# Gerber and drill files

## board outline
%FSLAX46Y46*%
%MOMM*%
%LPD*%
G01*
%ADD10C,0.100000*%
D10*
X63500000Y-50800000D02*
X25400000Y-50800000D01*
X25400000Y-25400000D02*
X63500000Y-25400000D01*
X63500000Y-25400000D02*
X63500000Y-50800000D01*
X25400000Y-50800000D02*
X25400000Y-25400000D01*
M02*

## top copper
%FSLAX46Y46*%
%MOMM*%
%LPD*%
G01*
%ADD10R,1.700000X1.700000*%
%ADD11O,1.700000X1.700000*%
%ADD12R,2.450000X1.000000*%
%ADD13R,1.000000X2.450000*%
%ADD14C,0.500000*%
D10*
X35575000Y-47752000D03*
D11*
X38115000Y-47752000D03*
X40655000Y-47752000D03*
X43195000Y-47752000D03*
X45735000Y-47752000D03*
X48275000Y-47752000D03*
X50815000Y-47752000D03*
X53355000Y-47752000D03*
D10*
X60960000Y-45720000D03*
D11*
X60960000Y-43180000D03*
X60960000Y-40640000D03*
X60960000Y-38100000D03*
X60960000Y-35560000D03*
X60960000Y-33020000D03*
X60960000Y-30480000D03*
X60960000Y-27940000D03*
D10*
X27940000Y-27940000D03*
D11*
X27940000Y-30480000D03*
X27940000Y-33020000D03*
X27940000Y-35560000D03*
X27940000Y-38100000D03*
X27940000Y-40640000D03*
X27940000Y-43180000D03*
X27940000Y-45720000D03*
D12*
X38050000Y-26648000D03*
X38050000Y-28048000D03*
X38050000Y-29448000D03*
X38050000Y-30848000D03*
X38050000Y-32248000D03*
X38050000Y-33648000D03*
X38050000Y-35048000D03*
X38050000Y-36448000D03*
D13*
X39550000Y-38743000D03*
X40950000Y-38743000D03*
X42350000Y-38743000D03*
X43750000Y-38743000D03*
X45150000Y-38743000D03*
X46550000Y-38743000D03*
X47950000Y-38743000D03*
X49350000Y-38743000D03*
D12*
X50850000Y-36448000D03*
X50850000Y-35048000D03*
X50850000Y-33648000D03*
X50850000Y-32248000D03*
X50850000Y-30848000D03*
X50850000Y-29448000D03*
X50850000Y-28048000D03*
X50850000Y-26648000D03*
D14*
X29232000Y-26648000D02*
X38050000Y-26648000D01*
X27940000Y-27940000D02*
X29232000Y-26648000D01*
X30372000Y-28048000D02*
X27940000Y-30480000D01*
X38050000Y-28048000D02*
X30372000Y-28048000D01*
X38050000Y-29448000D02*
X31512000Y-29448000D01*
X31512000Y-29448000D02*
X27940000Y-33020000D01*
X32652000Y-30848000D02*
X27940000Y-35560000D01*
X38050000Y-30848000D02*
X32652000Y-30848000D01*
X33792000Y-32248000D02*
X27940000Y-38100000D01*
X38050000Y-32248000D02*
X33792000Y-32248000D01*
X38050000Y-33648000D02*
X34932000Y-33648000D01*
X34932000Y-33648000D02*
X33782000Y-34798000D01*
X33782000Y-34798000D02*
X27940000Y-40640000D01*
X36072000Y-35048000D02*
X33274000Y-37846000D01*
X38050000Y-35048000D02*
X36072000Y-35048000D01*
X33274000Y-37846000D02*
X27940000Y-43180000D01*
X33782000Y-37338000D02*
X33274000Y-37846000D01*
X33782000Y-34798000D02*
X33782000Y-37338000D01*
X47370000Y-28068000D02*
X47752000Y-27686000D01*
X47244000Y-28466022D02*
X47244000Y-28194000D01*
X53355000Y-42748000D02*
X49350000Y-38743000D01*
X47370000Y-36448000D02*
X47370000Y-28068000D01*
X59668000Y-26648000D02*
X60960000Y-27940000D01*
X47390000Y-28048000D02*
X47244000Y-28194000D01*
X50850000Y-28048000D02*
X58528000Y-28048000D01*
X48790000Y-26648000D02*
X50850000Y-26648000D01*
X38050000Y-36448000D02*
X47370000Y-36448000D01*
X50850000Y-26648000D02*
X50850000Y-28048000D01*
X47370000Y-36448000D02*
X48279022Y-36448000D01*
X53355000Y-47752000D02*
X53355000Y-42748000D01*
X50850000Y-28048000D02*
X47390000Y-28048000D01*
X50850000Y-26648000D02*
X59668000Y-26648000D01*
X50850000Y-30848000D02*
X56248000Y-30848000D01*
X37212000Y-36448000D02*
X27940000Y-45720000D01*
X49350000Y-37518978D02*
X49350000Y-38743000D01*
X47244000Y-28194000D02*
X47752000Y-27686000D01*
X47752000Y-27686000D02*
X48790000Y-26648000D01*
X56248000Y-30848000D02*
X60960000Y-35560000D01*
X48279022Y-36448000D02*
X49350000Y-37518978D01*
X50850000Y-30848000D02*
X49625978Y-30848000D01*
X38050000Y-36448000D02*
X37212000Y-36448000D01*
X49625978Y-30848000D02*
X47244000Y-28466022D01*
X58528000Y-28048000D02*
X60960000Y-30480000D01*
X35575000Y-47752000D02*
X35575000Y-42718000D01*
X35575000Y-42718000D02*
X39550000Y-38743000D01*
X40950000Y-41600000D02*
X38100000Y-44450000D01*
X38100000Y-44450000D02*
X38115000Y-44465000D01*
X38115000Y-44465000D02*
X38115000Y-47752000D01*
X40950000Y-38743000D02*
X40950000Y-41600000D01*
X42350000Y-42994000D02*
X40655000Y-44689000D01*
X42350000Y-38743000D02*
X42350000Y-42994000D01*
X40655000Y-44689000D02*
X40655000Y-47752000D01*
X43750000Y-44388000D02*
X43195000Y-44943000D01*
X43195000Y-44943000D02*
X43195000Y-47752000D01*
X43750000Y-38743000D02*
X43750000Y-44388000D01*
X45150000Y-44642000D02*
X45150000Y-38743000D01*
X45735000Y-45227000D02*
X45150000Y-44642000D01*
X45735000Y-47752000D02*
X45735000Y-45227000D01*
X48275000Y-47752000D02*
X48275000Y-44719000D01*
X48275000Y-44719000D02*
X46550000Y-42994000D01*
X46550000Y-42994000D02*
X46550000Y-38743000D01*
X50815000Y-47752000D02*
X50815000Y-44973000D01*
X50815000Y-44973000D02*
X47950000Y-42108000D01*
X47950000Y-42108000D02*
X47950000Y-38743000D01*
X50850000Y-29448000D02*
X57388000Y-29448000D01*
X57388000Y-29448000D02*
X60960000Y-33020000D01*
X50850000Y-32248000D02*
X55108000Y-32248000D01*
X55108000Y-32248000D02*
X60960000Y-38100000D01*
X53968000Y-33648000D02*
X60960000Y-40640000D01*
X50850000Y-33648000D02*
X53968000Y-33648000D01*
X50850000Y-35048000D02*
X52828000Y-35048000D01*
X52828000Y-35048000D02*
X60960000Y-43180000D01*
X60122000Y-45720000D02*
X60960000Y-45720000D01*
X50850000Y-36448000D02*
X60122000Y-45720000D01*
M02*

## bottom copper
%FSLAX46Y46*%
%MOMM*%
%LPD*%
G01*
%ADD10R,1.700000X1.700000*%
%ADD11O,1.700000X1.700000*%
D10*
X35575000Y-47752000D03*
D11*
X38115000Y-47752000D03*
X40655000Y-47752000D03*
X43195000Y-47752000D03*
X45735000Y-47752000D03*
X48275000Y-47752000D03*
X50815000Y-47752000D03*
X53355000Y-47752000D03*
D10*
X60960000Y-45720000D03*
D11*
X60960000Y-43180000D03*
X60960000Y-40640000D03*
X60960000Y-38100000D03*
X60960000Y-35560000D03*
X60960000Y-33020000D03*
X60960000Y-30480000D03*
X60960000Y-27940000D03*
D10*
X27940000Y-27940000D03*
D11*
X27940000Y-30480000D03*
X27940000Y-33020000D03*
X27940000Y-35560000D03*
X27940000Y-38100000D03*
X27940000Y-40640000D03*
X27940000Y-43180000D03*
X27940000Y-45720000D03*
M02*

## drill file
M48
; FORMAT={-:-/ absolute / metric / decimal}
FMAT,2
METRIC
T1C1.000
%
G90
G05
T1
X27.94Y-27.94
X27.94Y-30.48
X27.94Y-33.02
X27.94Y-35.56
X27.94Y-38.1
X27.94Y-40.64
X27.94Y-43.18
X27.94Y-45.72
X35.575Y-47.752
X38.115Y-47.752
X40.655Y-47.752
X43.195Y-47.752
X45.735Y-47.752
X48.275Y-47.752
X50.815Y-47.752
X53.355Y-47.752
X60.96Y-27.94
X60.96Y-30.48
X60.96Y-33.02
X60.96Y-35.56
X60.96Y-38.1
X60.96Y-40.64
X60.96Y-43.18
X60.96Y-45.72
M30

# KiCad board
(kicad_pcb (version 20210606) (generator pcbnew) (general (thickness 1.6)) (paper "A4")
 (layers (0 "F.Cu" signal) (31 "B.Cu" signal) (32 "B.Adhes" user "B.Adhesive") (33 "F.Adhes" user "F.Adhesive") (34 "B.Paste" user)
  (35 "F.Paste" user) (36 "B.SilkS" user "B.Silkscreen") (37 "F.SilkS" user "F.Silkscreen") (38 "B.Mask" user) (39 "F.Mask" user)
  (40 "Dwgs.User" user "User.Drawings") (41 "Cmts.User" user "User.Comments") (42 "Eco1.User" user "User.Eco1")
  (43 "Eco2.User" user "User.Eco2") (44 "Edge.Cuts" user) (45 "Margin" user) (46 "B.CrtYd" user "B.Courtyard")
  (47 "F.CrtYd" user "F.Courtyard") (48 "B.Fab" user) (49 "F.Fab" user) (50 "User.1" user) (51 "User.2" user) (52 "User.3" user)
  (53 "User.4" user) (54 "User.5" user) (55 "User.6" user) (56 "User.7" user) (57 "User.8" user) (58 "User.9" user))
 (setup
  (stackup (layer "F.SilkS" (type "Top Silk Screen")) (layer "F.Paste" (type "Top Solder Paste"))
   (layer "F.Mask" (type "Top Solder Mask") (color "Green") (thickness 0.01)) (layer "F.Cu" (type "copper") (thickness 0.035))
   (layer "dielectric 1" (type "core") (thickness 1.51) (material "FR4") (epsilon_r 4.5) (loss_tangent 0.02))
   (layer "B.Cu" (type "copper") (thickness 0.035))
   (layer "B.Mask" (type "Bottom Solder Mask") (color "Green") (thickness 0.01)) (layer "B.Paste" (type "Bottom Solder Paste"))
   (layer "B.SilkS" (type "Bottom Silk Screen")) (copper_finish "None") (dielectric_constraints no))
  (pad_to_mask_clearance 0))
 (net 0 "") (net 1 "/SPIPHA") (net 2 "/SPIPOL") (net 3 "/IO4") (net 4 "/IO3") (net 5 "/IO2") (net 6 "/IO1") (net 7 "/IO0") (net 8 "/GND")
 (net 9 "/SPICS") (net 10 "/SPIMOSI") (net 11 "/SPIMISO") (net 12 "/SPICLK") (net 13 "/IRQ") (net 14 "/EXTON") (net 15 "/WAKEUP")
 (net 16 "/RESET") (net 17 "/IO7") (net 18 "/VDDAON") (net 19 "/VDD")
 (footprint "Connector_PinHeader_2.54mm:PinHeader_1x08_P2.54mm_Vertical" (layer "F.Cu") (at 35.575 47.752 90)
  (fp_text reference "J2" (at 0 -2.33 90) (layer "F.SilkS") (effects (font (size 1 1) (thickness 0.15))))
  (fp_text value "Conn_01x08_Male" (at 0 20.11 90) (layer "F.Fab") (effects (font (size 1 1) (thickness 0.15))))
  (pad "1" thru_hole rect locked (at 0 0 90) (size 1.7 1.7) (drill 1) (layers *.Cu *.Mask) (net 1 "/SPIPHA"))
  (pad "2" thru_hole oval locked (at 0 2.54 90) (size 1.7 1.7) (drill 1) (layers *.Cu *.Mask) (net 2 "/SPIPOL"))
  (pad "3" thru_hole oval locked (at 0 5.08 90) (size 1.7 1.7) (drill 1) (layers *.Cu *.Mask) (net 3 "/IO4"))
  (pad "4" thru_hole oval locked (at 0 7.62 90) (size 1.7 1.7) (drill 1) (layers *.Cu *.Mask) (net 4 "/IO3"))
  (pad "5" thru_hole oval locked (at 0 10.16 90) (size 1.7 1.7) (drill 1) (layers *.Cu *.Mask) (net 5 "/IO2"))
  (pad "6" thru_hole oval locked (at 0 12.7 90) (size 1.7 1.7) (drill 1) (layers *.Cu *.Mask) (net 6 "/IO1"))
  (pad "7" thru_hole oval locked (at 0 15.24 90) (size 1.7 1.7) (drill 1) (layers *.Cu *.Mask) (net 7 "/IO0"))
  (pad "8" thru_hole oval locked (at 0 17.78 90) (size 1.7 1.7) (drill 1) (layers *.Cu *.Mask) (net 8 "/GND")))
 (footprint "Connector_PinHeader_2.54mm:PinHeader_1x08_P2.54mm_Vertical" (layer "F.Cu") (at 60.96 45.72 180)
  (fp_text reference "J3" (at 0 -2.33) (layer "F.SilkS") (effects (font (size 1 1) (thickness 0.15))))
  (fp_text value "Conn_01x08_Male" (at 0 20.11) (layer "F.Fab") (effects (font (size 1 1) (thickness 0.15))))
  (pad "1" thru_hole rect locked (at 0 0 180) (size 1.7 1.7) (drill 1) (layers *.Cu *.Mask) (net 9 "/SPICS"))
  (pad "2" thru_hole oval locked (at 0 2.54 180) (size 1.7 1.7) (drill 1) (layers *.Cu *.Mask) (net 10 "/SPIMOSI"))
  (pad "3" thru_hole oval locked (at 0 5.08 180) (size 1.7 1.7) (drill 1) (layers *.Cu *.Mask) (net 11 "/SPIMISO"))
  (pad "4" thru_hole oval locked (at 0 7.62 180) (size 1.7 1.7) (drill 1) (layers *.Cu *.Mask) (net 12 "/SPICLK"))
  (pad "5" thru_hole oval locked (at 0 10.16 180) (size 1.7 1.7) (drill 1) (layers *.Cu *.Mask) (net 8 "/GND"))
  (pad "6" thru_hole oval locked (at 0 12.7 180) (size 1.7 1.7) (drill 1) (layers *.Cu *.Mask) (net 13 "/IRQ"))
  (pad "7" thru_hole oval locked (at 0 15.24 180) (size 1.7 1.7) (drill 1) (layers *.Cu *.Mask) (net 8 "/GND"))
  (pad "8" thru_hole oval locked (at 0 17.78 180) (size 1.7 1.7) (drill 1) (layers *.Cu *.Mask) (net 8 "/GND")))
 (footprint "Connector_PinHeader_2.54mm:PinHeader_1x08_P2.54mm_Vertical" (layer "F.Cu") (at 27.94 27.94)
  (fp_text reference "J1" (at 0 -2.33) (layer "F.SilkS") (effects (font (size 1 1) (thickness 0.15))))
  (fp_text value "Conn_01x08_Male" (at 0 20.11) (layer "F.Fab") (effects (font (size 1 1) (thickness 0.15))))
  (pad "1" thru_hole rect locked (at 0 0) (size 1.7 1.7) (drill 1) (layers *.Cu *.Mask) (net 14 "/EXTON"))
  (pad "2" thru_hole oval locked (at 0 2.54) (size 1.7 1.7) (drill 1) (layers *.Cu *.Mask) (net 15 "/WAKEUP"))
  (pad "3" thru_hole oval locked (at 0 5.08) (size 1.7 1.7) (drill 1) (layers *.Cu *.Mask) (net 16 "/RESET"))
  (pad "4" thru_hole oval locked (at 0 7.62) (size 1.7 1.7) (drill 1) (layers *.Cu *.Mask) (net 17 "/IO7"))
  (pad "5" thru_hole oval locked (at 0 10.16) (size 1.7 1.7) (drill 1) (layers *.Cu *.Mask) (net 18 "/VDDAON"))
  (pad "6" thru_hole oval locked (at 0 12.7) (size 1.7 1.7) (drill 1) (layers *.Cu *.Mask) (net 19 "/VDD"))
  (pad "7" thru_hole oval locked (at 0 15.24) (size 1.7 1.7) (drill 1) (layers *.Cu *.Mask) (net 19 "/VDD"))
  (pad "8" thru_hole oval locked (at 0 17.78) (size 1.7 1.7) (drill 1) (layers *.Cu *.Mask) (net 8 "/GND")))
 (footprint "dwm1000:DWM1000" (layer "F.Cu") (at 44.45 28.448)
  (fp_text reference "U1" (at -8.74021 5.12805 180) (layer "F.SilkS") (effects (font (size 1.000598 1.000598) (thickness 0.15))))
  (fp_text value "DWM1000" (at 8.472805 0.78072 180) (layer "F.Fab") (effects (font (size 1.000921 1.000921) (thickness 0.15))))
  (pad "1" smd rect locked (at -6.4 -1.8) (size 2.45 1) (layers "F.Cu" "F.Paste" "F.Mask") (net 14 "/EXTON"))
  (pad "2" smd rect locked (at -6.4 -0.4) (size 2.45 1) (layers "F.Cu" "F.Paste" "F.Mask") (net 15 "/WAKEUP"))
  (pad "3" smd rect locked (at -6.4 1) (size 2.45 1) (layers "F.Cu" "F.Paste" "F.Mask") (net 16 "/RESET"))
  (pad "4" smd rect locked (at -6.4 2.4) (size 2.45 1) (layers "F.Cu" "F.Paste" "F.Mask") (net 17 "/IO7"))
  (pad "5" smd rect locked (at -6.4 3.8) (size 2.45 1) (layers "F.Cu" "F.Paste" "F.Mask") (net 18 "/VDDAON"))
  (pad "6" smd rect locked (at -6.4 5.2) (size 2.45 1) (layers "F.Cu" "F.Paste" "F.Mask") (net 19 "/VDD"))
  (pad "7" smd rect locked (at -6.4 6.6) (size 2.45 1) (layers "F.Cu" "F.Paste" "F.Mask") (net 19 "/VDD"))
  (pad "8" smd rect locked (at -6.4 8) (size 2.45 1) (layers "F.Cu" "F.Paste" "F.Mask") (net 8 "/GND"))
  (pad "9" smd rect locked (at -4.9 10.295) (size 1 2.45) (layers "F.Cu" "F.Paste" "F.Mask") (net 1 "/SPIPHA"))
  (pad "10" smd rect locked (at -3.5 10.295) (size 1 2.45) (layers "F.Cu" "F.Paste" "F.Mask") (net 2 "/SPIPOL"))
  (pad "11" smd rect locked (at -2.1 10.295) (size 1 2.45) (layers "F.Cu" "F.Paste" "F.Mask") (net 3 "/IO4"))
  (pad "12" smd rect locked (at -0.7 10.295) (size 1 2.45) (layers "F.Cu" "F.Paste" "F.Mask") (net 4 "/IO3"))
  (pad "13" smd rect locked (at 0.7 10.295) (size 1 2.45) (layers "F.Cu" "F.Paste" "F.Mask") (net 5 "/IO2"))
  (pad "14" smd rect locked (at 2.1 10.295) (size 1 2.45) (layers "F.Cu" "F.Paste" "F.Mask") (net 6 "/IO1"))
  (pad "15" smd rect locked (at 3.5 10.295) (size 1 2.45) (layers "F.Cu" "F.Paste" "F.Mask") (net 7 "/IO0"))
  (pad "16" smd rect locked (at 4.9 10.295) (size 1 2.45) (layers "F.Cu" "F.Paste" "F.Mask") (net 8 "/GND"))
  (pad "17" smd rect locked (at 6.4 8) (size 2.45 1) (layers "F.Cu" "F.Paste" "F.Mask") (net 9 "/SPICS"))
  (pad "18" smd rect locked (at 6.4 6.6) (size 2.45 1) (layers "F.Cu" "F.Paste" "F.Mask") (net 10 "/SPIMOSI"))
  (pad "19" smd rect locked (at 6.4 5.2) (size 2.45 1) (layers "F.Cu" "F.Paste" "F.Mask") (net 11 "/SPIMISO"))
  (pad "20" smd rect locked (at 6.4 3.8) (size 2.45 1) (layers "F.Cu" "F.Paste" "F.Mask") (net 12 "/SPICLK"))
  (pad "21" smd rect locked (at 6.4 2.4) (size 2.45 1) (layers "F.Cu" "F.Paste" "F.Mask") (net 8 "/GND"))
  (pad "22" smd rect locked (at 6.4 1) (size 2.45 1) (layers "F.Cu" "F.Paste" "F.Mask") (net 13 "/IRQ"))
  (pad "23" smd rect locked (at 6.4 -0.4) (size 2.45 1) (layers "F.Cu" "F.Paste" "F.Mask") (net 8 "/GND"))
  (pad "24" smd rect locked (at 6.4 -1.8) (size 2.45 1) (layers "F.Cu" "F.Paste" "F.Mask") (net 8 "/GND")))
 (gr_line (start 63.5 50.8) (end 25.4 50.8) (layer "Edge.Cuts") (width 0.1))
 (gr_line (start 25.4 25.4) (end 63.5 25.4) (layer "Edge.Cuts") (width 0.1))
 (gr_line (start 63.5 25.4) (end 63.5 50.8) (layer "Edge.Cuts") (width 0.1))
 (gr_line (start 25.4 50.8) (end 25.4 25.4) (layer "Edge.Cuts") (width 0.1))
 (segment (start 29.232 26.648) (end 38.05 26.648) (width 0.5) (layer "F.Cu") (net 14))
 (segment (start 27.94 27.94) (end 29.232 26.648) (width 0.5) (layer "F.Cu") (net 14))
 (segment (start 30.372 28.048) (end 27.94 30.48) (width 0.5) (layer "F.Cu") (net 15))
 (segment (start 38.05 28.048) (end 30.372 28.048) (width 0.5) (layer "F.Cu") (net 15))
 (segment (start 38.05 29.448) (end 31.512 29.448) (width 0.5) (layer "F.Cu") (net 16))
 (segment (start 31.512 29.448) (end 27.94 33.02) (width 0.5) (layer "F.Cu") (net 16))
 (segment (start 32.652 30.848) (end 27.94 35.56) (width 0.5) (layer "F.Cu") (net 17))
 (segment (start 38.05 30.848) (end 32.652 30.848) (width 0.5) (layer "F.Cu") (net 17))
 (segment (start 33.792 32.248) (end 27.94 38.1) (width 0.5) (layer "F.Cu") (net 18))
 (segment (start 38.05 32.248) (end 33.792 32.248) (width 0.5) (layer "F.Cu") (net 18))
 (segment (start 38.05 33.648) (end 34.932 33.648) (width 0.5) (layer "F.Cu") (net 19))
 (segment (start 34.932 33.648) (end 33.782 34.798) (width 0.5) (layer "F.Cu") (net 19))
 (segment (start 33.782 34.798) (end 27.94 40.64) (width 0.5) (layer "F.Cu") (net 19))
 (segment (start 36.072 35.048) (end 33.274 37.846) (width 0.5) (layer "F.Cu") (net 19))
 (segment (start 38.05 35.048) (end 36.072 35.048) (width 0.5) (layer "F.Cu") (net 19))
 (segment (start 33.274 37.846) (end 27.94 43.18) (width 0.5) (layer "F.Cu") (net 19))
 (segment (start 33.782 37.338) (end 33.274 37.846) (width 0.5) (layer "F.Cu") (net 19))
 (segment (start 33.782 34.798) (end 33.782 37.338) (width 0.5) (layer "F.Cu") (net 19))
 (segment (start 47.37 28.068) (end 47.752 27.686) (width 0.5) (layer "F.Cu") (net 8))
 (segment (start 47.244 28.466022) (end 47.244 28.194) (width 0.5) (layer "F.Cu") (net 8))
 (segment (start 53.355 42.748) (end 49.35 38.743) (width 0.5) (layer "F.Cu") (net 8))
 (segment (start 47.37 36.448) (end 47.37 28.068) (width 0.5) (layer "F.Cu") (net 8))
 (segment (start 59.668 26.648) (end 60.96 27.94) (width 0.5) (layer "F.Cu") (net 8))
 (segment (start 47.39 28.048) (end 47.244 28.194) (width 0.5) (layer "F.Cu") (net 8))
 (segment (start 50.85 28.048) (end 58.528 28.048) (width 0.5) (layer "F.Cu") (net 8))
 (segment (start 48.79 26.648) (end 50.85 26.648) (width 0.5) (layer "F.Cu") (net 8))
 (segment (start 38.05 36.448) (end 47.37 36.448) (width 0.5) (layer "F.Cu") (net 8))
 (segment (start 50.85 26.648) (end 50.85 28.048) (width 0.5) (layer "F.Cu") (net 8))
 (segment (start 47.37 36.448) (end 48.279022 36.448) (width 0.5) (layer "F.Cu") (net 8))
 (segment (start 53.355 47.752) (end 53.355 42.748) (width 0.5) (layer "F.Cu") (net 8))
 (segment (start 50.85 28.048) (end 47.39 28.048) (width 0.5) (layer "F.Cu") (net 8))
 (segment (start 50.85 26.648) (end 59.668 26.648) (width 0.5) (layer "F.Cu") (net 8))
 (segment (start 50.85 30.848) (end 56.248 30.848) (width 0.5) (layer "F.Cu") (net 8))
 (segment (start 37.212 36.448) (end 27.94 45.72) (width 0.5) (layer "F.Cu") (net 8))
 (segment (start 49.35 37.518978) (end 49.35 38.743) (width 0.5) (layer "F.Cu") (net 8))
 (segment (start 47.244 28.194) (end 47.752 27.686) (width 0.5) (layer "F.Cu") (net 8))
 (segment (start 47.752 27.686) (end 48.79 26.648) (width 0.5) (layer "F.Cu") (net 8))
 (segment (start 56.248 30.848) (end 60.96 35.56) (width 0.5) (layer "F.Cu") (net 8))
 (segment (start 48.279022 36.448) (end 49.35 37.518978) (width 0.5) (layer "F.Cu") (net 8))
 (segment (start 50.85 30.848) (end 49.625978 30.848) (width 0.5) (layer "F.Cu") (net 8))
 (segment (start 38.05 36.448) (end 37.212 36.448) (width 0.5) (layer "F.Cu") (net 8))
 (segment (start 49.625978 30.848) (end 47.244 28.466022) (width 0.5) (layer "F.Cu") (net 8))
 (segment (start 58.528 28.048) (end 60.96 30.48) (width 0.5) (layer "F.Cu") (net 8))
 (segment (start 35.575 47.752) (end 35.575 42.718) (width 0.5) (layer "F.Cu") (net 1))
 (segment (start 35.575 42.718) (end 39.55 38.743) (width 0.5) (layer "F.Cu") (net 1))
 (segment (start 40.95 41.6) (end 38.1 44.45) (width 0.5) (layer "F.Cu") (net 2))
 (segment (start 38.1 44.45) (end 38.115 44.465) (width 0.5) (layer "F.Cu") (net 2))
 (segment (start 38.115 44.465) (end 38.115 47.752) (width 0.5) (layer "F.Cu") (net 2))
 (segment (start 40.95 38.743) (end 40.95 41.6) (width 0.5) (layer "F.Cu") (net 2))
 (segment (start 42.35 42.994) (end 40.655 44.689) (width 0.5) (layer "F.Cu") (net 3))
 (segment (start 42.35 38.743) (end 42.35 42.994) (width 0.5) (layer "F.Cu") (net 3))
 (segment (start 40.655 44.689) (end 40.655 47.752) (width 0.5) (layer "F.Cu") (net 3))
 (segment (start 43.75 44.388) (end 43.195 44.943) (width 0.5) (layer "F.Cu") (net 4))
 (segment (start 43.195 44.943) (end 43.195 47.752) (width 0.5) (layer "F.Cu") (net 4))
 (segment (start 43.75 38.743) (end 43.75 44.388) (width 0.5) (layer "F.Cu") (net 4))
 (segment (start 45.15 44.642) (end 45.15 38.743) (width 0.5) (layer "F.Cu") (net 5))
 (segment (start 45.735 45.227) (end 45.15 44.642) (width 0.5) (layer "F.Cu") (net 5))
 (segment (start 45.735 47.752) (end 45.735 45.227) (width 0.5) (layer "F.Cu") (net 5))
 (segment (start 48.275 47.752) (end 48.275 44.719) (width 0.5) (layer "F.Cu") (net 6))
 (segment (start 48.275 44.719) (end 46.55 42.994) (width 0.5) (layer "F.Cu") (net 6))
 (segment (start 46.55 42.994) (end 46.55 38.743) (width 0.5) (layer "F.Cu") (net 6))
 (segment (start 50.815 47.752) (end 50.815 44.973) (width 0.5) (layer "F.Cu") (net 7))
 (segment (start 50.815 44.973) (end 47.95 42.108) (width 0.5) (layer "F.Cu") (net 7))
 (segment (start 47.95 42.108) (end 47.95 38.743) (width 0.5) (layer "F.Cu") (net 7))
 (segment (start 50.85 29.448) (end 57.388 29.448) (width 0.5) (layer "F.Cu") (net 13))
 (segment (start 57.388 29.448) (end 60.96 33.02) (width 0.5) (layer "F.Cu") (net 13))
 (segment (start 50.85 32.248) (end 55.108 32.248) (width 0.5) (layer "F.Cu") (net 12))
 (segment (start 55.108 32.248) (end 60.96 38.1) (width 0.5) (layer "F.Cu") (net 12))
 (segment (start 53.968 33.648) (end 60.96 40.64) (width 0.5) (layer "F.Cu") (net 11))
 (segment (start 50.85 33.648) (end 53.968 33.648) (width 0.5) (layer "F.Cu") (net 11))
 (segment (start 50.85 35.048) (end 52.828 35.048) (width 0.5) (layer "F.Cu") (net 10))
 (segment (start 52.828 35.048) (end 60.96 43.18) (width 0.5) (layer "F.Cu") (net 10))
 (segment (start 60.122 45.72) (end 60.96 45.72) (width 0.5) (layer "F.Cu") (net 9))
 (segment (start 50.85 36.448) (end 60.122 45.72) (width 0.5) (layer "F.Cu") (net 9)))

